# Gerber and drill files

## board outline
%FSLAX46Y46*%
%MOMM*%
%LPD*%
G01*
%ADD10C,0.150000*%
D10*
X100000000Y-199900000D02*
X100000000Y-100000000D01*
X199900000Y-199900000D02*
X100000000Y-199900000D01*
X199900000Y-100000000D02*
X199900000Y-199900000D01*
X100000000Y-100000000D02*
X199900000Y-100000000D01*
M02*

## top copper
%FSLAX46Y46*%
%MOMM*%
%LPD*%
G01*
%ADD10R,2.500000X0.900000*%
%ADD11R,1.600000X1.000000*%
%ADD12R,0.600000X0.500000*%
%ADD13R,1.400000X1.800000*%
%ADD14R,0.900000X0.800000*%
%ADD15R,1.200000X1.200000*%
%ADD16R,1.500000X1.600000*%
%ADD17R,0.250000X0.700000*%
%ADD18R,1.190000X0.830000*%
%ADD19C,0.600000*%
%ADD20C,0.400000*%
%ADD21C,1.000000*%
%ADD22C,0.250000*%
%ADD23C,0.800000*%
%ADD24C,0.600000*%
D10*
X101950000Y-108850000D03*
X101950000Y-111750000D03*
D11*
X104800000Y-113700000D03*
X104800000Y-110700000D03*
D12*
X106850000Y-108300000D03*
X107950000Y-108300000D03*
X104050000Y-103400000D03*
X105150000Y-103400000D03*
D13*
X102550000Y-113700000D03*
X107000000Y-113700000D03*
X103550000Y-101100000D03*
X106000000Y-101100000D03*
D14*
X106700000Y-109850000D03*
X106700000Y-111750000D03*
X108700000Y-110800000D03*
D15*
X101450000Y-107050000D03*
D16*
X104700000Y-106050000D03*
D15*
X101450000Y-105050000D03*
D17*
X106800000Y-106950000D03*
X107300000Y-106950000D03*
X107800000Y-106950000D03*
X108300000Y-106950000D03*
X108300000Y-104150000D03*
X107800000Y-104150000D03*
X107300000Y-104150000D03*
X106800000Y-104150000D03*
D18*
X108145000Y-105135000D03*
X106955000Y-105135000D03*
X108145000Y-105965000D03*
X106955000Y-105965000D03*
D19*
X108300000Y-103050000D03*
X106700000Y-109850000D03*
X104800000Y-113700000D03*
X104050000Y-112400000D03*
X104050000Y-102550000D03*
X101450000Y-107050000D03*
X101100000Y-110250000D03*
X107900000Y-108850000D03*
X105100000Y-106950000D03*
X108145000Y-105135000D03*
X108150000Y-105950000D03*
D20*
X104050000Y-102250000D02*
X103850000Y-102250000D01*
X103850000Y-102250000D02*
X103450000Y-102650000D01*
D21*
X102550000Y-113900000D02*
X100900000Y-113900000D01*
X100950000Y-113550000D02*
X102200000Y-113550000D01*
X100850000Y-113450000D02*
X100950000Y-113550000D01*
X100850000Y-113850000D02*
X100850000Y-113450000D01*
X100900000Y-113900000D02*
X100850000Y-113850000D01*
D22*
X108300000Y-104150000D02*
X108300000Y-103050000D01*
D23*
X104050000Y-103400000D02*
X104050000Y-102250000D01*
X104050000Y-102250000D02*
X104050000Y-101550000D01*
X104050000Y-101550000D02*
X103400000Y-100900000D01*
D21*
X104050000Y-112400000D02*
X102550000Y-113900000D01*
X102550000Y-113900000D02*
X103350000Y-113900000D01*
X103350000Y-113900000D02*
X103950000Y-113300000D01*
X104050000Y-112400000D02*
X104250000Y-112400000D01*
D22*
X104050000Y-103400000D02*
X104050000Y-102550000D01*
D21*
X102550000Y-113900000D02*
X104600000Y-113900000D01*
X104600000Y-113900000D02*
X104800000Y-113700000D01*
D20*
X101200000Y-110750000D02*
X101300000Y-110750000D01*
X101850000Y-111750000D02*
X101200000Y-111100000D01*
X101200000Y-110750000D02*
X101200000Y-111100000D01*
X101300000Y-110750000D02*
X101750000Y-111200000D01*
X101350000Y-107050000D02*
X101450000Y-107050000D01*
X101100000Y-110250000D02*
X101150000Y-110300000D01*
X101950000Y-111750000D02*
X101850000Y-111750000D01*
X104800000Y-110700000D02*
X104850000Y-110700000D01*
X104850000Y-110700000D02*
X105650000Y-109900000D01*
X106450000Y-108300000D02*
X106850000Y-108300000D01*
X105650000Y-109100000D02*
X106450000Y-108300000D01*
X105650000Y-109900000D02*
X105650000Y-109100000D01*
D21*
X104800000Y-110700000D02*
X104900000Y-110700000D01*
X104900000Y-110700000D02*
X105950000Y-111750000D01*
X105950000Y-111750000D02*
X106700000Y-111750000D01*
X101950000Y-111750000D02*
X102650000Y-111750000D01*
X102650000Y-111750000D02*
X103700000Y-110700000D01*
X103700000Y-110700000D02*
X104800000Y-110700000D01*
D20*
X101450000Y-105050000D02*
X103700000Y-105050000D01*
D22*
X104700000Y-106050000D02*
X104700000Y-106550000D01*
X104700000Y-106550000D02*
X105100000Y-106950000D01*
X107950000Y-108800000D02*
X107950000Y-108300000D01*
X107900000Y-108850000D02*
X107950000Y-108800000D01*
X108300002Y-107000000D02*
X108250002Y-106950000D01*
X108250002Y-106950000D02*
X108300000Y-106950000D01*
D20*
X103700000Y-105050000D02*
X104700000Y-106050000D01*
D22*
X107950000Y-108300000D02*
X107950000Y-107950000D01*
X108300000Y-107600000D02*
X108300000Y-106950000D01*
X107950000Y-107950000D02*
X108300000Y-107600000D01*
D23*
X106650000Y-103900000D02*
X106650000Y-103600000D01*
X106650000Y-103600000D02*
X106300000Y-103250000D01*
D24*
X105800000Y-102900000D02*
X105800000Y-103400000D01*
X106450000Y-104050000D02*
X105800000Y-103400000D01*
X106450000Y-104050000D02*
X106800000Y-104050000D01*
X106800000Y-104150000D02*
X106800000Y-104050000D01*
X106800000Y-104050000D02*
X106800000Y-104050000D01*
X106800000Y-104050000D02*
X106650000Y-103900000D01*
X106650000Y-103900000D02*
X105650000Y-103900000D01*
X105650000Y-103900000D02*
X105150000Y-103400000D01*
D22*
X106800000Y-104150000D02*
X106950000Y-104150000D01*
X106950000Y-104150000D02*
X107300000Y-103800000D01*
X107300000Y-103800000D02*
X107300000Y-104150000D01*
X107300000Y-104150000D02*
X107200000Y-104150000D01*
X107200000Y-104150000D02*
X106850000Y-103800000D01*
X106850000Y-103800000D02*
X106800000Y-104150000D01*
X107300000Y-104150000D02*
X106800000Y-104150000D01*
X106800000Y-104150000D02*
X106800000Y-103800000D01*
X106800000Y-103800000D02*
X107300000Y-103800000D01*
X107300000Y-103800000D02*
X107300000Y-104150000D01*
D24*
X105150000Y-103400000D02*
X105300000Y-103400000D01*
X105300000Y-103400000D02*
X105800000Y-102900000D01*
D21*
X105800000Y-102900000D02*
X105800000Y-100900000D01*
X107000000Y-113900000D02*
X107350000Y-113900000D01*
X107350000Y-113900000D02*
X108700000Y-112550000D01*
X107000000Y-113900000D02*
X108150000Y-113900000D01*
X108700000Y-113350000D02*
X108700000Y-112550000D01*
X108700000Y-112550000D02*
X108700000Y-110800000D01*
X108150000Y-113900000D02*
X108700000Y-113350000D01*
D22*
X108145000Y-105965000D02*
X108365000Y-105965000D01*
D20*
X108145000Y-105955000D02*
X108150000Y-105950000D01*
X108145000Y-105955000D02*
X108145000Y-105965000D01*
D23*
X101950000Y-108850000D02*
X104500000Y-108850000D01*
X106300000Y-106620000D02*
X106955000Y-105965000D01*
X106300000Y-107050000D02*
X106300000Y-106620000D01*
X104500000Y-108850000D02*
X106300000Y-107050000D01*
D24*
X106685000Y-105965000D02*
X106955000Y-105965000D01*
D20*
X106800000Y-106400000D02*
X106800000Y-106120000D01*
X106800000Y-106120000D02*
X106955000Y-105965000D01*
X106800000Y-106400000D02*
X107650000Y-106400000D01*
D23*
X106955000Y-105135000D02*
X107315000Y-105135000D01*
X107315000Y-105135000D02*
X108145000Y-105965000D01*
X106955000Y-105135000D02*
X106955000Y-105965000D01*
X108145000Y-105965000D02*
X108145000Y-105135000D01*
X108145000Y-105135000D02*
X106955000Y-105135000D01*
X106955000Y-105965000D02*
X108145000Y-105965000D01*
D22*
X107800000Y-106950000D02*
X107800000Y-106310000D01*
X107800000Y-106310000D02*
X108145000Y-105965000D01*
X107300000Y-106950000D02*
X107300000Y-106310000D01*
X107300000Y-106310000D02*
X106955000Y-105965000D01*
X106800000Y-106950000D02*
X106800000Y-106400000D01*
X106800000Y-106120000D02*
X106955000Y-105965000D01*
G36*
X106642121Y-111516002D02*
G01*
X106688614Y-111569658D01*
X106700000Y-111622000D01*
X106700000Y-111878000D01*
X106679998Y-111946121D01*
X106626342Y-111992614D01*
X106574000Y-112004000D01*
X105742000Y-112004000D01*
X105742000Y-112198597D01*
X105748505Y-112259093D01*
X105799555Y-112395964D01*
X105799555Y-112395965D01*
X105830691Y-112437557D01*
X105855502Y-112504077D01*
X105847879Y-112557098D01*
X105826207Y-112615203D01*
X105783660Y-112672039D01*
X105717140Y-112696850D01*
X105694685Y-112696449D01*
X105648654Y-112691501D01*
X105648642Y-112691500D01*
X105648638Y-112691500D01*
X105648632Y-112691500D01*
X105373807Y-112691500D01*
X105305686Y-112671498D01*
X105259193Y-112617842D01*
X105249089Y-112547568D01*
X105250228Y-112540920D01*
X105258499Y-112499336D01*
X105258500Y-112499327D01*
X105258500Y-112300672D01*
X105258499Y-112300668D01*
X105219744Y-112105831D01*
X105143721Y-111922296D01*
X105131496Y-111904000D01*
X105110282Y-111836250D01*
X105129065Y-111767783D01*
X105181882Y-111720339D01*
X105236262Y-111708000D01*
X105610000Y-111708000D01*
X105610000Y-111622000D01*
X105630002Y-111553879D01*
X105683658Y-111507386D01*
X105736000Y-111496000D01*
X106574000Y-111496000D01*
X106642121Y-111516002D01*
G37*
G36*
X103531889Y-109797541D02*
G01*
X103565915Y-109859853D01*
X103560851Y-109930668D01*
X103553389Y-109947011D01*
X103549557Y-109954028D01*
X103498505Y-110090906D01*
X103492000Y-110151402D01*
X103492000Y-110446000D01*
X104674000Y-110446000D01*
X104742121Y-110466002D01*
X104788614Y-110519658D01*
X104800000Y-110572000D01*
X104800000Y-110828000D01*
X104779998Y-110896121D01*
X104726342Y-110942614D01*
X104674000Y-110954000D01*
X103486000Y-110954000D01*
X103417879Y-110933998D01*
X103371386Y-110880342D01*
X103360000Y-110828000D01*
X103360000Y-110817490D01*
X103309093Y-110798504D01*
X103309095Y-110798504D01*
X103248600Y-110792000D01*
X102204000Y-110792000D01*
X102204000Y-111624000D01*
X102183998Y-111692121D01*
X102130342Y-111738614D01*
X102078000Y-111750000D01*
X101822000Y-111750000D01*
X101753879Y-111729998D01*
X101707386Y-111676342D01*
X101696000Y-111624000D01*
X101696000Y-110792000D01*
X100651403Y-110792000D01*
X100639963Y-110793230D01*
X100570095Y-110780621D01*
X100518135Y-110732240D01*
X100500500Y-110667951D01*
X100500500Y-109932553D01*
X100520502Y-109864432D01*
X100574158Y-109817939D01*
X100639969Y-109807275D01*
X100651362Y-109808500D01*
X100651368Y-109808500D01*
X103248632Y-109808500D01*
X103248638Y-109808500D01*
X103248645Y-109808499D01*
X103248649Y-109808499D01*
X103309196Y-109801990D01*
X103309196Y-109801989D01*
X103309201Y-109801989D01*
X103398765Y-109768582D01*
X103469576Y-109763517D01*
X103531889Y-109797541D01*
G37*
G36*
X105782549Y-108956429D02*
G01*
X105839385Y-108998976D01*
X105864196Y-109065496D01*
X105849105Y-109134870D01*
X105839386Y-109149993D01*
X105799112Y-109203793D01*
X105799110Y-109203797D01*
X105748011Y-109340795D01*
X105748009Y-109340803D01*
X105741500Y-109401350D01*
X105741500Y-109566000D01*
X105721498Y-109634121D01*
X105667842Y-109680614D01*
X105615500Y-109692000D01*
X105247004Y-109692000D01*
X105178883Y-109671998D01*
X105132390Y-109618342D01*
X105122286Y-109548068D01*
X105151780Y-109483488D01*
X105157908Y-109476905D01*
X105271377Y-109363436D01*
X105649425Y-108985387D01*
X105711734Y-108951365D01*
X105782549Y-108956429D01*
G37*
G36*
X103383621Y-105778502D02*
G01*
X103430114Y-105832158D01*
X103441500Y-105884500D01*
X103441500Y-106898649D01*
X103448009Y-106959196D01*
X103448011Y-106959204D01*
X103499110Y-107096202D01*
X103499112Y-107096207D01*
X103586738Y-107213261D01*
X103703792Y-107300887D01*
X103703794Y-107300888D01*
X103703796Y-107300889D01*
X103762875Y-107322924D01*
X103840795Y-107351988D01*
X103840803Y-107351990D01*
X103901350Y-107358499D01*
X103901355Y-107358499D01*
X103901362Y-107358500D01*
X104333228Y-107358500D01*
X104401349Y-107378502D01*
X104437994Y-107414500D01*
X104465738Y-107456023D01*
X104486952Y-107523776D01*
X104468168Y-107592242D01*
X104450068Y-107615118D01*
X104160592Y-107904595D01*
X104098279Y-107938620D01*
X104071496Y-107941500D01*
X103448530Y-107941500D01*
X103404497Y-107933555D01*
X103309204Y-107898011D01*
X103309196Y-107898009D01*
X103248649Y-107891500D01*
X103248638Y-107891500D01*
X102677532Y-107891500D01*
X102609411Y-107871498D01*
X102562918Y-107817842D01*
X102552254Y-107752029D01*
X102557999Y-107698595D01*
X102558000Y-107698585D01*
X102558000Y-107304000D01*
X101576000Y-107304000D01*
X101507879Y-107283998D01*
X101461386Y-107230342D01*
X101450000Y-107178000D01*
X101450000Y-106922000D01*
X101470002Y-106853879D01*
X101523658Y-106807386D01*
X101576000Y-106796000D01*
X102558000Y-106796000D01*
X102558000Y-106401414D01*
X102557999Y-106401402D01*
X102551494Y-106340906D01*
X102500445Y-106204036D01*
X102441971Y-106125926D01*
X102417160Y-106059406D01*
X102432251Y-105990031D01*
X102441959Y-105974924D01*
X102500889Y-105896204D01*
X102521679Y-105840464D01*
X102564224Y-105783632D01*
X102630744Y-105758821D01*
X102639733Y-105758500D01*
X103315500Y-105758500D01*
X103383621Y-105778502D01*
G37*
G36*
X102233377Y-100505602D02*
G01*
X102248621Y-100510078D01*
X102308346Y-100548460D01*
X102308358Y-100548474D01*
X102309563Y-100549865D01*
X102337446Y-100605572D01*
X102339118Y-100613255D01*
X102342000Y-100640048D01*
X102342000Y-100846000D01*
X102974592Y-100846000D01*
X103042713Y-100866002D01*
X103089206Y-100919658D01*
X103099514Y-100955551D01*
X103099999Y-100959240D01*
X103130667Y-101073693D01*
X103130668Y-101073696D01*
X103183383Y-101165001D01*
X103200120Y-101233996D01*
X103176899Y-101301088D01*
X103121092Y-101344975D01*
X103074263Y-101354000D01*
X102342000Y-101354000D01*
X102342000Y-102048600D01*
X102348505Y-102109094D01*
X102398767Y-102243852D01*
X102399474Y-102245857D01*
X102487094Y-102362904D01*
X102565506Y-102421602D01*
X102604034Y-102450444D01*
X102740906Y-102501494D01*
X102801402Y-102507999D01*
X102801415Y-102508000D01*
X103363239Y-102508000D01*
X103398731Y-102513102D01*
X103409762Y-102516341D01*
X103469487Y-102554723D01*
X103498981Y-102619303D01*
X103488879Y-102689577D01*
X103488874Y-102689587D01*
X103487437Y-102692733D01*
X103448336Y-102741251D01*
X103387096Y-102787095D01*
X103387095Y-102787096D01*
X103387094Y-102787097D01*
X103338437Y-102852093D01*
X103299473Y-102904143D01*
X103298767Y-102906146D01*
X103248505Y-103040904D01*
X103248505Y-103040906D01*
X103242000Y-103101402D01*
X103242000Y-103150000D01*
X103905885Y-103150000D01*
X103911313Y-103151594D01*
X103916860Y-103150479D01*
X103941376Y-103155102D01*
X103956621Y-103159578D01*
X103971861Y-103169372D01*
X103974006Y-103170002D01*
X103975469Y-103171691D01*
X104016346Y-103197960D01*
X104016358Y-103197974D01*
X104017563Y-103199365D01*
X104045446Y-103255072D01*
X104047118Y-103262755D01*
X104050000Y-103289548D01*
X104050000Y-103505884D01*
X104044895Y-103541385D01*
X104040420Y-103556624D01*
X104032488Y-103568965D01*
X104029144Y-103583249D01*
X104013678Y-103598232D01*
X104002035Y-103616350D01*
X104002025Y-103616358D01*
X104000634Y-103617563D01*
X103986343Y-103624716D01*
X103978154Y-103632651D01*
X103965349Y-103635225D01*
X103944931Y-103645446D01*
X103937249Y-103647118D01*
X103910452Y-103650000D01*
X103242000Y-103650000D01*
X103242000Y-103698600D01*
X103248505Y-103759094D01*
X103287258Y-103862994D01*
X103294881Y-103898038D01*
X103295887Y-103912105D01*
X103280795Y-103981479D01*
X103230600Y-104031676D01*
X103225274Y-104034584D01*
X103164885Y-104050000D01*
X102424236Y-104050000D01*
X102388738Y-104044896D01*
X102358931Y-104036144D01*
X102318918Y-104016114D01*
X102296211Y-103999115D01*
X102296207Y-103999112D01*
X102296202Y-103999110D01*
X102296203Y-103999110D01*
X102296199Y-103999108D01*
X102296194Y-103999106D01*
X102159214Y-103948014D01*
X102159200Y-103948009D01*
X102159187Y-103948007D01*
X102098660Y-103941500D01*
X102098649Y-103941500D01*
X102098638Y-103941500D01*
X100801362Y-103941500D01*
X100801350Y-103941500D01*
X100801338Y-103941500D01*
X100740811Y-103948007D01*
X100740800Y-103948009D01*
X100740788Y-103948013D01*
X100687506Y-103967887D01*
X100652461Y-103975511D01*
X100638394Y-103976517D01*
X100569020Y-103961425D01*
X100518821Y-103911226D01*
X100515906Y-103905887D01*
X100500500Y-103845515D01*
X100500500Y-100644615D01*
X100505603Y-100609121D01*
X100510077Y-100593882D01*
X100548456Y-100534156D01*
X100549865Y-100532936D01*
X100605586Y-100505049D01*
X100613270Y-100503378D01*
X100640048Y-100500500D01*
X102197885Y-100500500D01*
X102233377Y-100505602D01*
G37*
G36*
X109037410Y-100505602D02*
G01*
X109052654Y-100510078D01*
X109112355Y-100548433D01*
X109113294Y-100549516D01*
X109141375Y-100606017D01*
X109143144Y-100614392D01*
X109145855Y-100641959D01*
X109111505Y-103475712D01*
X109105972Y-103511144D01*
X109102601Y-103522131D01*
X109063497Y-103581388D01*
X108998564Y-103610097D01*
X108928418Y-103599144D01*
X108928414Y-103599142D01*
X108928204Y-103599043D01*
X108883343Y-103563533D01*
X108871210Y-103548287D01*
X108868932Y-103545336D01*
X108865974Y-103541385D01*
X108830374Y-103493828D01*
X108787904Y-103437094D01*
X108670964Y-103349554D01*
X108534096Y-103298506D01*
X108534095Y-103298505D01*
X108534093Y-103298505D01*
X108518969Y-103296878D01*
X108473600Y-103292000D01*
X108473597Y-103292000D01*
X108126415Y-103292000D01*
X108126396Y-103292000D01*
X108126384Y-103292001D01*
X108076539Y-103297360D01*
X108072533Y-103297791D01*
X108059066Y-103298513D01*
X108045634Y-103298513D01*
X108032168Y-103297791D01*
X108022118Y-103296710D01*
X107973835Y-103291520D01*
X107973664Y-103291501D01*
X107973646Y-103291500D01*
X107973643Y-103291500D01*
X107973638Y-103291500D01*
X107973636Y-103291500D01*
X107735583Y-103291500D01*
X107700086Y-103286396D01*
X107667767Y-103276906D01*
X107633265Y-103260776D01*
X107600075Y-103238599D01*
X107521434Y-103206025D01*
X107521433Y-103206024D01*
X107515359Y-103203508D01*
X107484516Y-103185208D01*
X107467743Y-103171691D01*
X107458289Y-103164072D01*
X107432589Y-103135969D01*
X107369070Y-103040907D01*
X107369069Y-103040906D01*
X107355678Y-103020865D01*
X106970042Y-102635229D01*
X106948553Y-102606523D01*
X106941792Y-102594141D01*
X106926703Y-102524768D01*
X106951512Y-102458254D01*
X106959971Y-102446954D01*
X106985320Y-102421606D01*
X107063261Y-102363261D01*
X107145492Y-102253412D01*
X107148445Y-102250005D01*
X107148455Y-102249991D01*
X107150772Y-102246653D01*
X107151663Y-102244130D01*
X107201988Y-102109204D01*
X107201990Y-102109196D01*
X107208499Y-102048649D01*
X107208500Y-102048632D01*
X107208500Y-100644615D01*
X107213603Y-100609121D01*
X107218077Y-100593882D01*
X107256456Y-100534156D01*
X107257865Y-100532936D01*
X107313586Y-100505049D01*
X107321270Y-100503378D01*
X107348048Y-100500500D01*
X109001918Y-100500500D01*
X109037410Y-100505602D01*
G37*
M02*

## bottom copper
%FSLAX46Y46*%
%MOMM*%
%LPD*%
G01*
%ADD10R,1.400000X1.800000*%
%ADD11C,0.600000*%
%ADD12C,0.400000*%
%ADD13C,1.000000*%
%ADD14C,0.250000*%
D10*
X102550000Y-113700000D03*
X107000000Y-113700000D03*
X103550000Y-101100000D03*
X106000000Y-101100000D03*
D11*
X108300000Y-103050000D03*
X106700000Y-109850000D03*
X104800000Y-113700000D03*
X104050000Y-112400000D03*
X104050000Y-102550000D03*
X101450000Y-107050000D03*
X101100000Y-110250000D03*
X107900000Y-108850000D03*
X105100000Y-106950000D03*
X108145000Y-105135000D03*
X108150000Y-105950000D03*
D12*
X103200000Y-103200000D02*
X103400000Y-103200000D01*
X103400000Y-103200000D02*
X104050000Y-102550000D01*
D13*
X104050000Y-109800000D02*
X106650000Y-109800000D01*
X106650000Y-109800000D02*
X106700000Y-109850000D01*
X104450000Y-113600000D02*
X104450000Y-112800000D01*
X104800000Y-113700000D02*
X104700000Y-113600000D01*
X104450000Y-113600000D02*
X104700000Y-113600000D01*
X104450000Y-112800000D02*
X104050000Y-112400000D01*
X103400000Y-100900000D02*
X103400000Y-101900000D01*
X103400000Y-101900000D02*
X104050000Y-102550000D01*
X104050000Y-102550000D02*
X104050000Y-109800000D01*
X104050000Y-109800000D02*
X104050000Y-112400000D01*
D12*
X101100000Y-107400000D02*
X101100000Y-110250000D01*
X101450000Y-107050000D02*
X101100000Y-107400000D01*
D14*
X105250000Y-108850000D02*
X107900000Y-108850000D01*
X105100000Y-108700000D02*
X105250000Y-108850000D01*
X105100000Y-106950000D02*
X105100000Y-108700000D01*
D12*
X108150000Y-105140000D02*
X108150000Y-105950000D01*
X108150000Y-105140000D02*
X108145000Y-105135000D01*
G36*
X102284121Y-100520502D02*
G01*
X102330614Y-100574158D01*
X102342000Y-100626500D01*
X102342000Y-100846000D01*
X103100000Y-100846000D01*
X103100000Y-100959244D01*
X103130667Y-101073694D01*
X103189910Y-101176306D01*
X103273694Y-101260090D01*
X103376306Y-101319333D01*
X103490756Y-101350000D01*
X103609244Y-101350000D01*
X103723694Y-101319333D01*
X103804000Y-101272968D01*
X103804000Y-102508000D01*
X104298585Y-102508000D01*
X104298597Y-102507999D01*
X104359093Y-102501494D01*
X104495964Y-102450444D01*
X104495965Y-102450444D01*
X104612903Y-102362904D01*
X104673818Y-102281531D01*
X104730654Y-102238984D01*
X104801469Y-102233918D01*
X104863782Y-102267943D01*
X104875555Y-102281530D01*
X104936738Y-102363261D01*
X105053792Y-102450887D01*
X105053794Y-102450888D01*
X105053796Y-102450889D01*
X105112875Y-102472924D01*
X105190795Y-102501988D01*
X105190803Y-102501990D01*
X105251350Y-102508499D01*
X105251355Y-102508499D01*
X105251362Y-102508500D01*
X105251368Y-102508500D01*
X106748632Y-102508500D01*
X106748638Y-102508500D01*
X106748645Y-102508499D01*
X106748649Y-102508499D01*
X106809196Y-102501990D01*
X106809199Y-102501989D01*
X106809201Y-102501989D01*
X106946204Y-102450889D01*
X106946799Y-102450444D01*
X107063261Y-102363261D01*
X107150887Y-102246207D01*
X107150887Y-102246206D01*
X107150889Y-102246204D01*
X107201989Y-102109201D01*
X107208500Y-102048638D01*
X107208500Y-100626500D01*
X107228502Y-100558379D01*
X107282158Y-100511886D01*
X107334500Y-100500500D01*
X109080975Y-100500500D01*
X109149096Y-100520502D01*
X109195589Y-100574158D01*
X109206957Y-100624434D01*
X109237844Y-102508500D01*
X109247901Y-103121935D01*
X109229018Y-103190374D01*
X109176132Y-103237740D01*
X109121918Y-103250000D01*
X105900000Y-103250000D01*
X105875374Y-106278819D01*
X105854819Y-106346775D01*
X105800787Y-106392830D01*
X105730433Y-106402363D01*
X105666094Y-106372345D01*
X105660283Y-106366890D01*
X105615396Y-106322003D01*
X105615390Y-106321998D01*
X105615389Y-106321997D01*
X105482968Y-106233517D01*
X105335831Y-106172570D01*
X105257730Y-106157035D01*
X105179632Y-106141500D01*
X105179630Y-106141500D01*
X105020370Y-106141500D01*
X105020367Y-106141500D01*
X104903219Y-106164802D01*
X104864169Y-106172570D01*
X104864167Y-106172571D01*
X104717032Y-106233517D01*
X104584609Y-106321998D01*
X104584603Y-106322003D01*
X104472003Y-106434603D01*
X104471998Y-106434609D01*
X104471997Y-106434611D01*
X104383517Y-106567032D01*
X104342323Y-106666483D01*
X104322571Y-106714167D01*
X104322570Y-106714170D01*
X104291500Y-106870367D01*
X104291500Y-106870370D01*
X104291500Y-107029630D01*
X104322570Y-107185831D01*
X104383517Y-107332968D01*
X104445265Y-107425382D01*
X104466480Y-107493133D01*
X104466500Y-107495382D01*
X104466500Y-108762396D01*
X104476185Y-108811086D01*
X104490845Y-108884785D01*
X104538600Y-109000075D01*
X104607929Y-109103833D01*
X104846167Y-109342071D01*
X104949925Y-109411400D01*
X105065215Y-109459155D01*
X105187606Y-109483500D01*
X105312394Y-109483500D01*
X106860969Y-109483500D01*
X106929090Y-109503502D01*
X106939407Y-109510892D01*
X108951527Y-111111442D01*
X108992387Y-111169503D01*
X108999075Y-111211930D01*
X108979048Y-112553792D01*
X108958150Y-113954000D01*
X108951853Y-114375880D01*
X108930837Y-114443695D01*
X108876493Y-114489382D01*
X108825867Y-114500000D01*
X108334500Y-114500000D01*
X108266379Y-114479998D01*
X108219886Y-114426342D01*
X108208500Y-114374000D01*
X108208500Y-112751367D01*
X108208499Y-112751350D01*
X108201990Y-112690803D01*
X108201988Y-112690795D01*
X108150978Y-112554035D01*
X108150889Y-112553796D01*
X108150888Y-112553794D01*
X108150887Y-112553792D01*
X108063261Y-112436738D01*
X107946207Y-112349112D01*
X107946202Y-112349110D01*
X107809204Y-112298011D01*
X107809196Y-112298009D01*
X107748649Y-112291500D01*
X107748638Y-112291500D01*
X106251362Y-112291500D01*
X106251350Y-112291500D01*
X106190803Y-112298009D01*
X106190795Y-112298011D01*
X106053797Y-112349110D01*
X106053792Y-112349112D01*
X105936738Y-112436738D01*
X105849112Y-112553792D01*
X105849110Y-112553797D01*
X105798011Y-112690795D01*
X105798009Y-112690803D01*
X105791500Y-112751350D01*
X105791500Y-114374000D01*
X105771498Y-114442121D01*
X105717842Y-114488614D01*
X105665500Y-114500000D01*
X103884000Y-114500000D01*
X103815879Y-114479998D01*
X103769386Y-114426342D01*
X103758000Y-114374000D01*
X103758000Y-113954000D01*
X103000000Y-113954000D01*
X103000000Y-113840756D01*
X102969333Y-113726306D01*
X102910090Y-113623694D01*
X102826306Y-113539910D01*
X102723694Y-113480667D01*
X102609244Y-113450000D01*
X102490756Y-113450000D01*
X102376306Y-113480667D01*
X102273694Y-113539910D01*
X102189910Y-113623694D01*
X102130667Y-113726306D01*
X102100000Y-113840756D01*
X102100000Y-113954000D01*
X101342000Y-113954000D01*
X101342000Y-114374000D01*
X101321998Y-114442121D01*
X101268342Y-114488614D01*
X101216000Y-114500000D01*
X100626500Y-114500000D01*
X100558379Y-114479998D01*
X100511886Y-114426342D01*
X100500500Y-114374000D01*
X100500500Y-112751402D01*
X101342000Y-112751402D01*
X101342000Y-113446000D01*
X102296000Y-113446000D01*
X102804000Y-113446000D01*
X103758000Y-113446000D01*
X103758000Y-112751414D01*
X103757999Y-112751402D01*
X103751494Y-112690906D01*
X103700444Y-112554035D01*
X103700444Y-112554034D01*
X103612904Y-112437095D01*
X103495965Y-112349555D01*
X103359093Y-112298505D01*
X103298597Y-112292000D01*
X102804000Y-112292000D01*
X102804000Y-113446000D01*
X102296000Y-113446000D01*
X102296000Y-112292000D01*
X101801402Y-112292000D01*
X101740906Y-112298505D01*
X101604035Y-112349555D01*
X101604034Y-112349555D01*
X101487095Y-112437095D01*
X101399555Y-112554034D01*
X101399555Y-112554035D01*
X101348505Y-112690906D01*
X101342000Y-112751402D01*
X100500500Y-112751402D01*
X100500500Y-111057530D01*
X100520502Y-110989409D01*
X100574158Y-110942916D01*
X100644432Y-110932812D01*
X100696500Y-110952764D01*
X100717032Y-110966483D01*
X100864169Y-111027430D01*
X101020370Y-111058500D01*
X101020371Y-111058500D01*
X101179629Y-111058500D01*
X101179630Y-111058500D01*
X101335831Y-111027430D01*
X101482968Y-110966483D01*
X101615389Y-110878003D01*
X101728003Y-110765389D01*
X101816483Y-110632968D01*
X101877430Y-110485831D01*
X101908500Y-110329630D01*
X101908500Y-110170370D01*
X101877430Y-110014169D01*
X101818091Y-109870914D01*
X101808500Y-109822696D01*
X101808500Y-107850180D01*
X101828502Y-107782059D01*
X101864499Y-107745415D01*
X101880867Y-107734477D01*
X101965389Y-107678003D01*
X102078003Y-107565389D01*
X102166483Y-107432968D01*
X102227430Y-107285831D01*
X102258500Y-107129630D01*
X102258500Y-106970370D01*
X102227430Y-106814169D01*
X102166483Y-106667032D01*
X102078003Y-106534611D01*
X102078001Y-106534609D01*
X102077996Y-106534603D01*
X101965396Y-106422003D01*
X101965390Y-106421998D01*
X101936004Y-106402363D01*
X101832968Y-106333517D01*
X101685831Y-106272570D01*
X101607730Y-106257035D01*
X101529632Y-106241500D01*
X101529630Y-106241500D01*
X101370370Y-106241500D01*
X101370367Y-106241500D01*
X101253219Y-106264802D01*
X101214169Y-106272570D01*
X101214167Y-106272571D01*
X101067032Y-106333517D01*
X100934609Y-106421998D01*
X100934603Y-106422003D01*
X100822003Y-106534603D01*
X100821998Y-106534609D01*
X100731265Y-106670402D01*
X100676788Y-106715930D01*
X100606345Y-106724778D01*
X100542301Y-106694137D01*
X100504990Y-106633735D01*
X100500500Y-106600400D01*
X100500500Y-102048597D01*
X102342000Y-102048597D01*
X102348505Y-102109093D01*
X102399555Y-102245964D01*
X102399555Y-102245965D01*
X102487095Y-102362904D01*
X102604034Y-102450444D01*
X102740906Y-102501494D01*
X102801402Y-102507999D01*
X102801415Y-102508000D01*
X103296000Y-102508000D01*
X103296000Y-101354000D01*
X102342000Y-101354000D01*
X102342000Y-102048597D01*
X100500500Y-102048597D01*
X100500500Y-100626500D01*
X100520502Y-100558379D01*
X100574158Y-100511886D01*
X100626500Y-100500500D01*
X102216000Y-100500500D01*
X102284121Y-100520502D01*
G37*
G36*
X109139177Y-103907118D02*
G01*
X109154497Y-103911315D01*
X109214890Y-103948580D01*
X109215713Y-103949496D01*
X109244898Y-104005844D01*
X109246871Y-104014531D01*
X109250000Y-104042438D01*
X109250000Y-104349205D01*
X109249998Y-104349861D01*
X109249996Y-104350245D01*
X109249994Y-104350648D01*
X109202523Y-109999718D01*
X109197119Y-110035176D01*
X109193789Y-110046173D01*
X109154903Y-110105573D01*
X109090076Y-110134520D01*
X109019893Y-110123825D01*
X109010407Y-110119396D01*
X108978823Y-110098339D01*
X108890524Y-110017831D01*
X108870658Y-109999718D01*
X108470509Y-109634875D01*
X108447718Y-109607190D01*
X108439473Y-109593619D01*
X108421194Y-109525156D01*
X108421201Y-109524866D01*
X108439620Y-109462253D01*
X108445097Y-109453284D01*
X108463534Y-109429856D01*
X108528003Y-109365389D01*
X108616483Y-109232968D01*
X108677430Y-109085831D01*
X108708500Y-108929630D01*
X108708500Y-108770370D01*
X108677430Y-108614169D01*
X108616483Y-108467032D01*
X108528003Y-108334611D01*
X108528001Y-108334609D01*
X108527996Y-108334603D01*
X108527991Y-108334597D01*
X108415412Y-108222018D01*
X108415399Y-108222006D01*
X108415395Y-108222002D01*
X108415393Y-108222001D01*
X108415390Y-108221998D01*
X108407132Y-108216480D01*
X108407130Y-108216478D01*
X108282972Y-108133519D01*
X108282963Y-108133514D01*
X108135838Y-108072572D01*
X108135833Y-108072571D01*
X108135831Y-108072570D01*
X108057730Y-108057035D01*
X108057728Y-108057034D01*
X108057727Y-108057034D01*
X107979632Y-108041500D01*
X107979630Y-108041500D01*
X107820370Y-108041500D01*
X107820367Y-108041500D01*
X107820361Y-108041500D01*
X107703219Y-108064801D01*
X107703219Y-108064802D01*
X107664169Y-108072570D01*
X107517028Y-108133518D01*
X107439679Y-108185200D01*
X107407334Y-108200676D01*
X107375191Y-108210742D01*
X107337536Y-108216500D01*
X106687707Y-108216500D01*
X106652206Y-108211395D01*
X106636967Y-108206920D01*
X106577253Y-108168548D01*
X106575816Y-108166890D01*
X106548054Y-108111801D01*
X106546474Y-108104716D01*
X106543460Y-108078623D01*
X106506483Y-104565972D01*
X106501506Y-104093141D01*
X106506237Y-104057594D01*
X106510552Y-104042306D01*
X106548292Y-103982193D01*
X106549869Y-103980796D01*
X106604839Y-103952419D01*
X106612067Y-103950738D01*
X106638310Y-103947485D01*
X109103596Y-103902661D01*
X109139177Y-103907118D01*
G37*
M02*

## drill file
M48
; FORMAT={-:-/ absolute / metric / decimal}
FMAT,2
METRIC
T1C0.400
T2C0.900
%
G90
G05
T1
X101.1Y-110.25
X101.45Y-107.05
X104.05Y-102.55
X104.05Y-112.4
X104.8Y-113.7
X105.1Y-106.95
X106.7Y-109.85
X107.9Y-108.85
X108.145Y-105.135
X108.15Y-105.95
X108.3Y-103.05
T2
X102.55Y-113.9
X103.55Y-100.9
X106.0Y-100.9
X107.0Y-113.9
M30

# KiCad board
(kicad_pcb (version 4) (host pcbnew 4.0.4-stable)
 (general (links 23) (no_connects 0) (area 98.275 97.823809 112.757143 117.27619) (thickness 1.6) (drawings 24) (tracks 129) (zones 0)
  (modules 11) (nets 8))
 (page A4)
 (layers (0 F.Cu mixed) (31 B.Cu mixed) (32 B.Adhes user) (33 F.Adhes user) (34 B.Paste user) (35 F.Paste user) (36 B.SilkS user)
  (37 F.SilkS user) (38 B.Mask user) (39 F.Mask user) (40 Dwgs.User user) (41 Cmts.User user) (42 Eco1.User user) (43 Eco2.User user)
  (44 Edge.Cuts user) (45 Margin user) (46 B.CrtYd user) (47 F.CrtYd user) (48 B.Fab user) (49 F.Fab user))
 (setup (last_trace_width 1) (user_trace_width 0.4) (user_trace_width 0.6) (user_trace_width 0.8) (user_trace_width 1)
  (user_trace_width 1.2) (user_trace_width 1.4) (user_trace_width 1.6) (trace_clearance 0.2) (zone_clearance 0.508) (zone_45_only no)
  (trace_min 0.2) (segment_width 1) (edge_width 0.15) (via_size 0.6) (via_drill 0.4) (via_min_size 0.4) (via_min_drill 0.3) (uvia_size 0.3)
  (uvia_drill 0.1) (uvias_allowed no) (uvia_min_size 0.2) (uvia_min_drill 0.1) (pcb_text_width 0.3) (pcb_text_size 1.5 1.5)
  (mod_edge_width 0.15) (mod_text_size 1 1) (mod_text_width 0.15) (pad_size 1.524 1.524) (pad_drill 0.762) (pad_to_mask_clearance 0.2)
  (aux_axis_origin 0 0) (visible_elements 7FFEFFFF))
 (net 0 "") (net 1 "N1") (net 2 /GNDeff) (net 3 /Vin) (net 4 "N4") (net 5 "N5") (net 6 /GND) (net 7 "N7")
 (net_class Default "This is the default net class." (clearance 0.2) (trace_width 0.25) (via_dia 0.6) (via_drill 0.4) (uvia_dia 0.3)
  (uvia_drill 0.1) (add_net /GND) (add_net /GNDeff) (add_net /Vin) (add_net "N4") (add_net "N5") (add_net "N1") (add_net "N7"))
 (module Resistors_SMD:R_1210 (layer F.Cu) (at 101.95 110.3 270)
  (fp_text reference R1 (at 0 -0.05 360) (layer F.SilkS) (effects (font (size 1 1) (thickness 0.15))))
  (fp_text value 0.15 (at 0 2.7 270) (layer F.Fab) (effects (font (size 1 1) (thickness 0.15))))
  (pad 1 smd rect (at -1.45 0 270) (size 0.9 2.5) (layers F.Cu F.Paste F.Mask) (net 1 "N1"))
  (pad 2 smd rect (at 1.45 0 270) (size 0.9 2.5) (layers F.Cu F.Paste F.Mask) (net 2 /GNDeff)))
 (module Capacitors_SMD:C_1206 (layer F.Cu) (at 104.8 112.2 90)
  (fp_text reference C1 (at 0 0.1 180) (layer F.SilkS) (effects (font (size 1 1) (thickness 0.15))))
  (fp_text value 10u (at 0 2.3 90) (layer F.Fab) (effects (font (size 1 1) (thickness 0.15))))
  (pad 1 smd rect (at -1.5 0 90) (size 1 1.6) (layers F.Cu F.Paste F.Mask) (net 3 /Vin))
  (pad 2 smd rect (at 1.5 0 90) (size 1 1.6) (layers F.Cu F.Paste F.Mask) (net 2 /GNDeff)))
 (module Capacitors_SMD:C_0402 (layer F.Cu) (at 107.4 108.3)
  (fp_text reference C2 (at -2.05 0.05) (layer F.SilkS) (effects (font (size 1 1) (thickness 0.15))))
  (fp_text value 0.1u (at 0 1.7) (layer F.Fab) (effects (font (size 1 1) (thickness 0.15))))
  (pad 1 smd rect (at -0.55 0) (size 0.6 0.5) (layers F.Cu F.Paste F.Mask) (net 2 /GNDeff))
  (pad 2 smd rect (at 0.55 0) (size 0.6 0.5) (layers F.Cu F.Paste F.Mask) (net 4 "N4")))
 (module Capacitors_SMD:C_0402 (layer F.Cu) (at 104.6 103.4)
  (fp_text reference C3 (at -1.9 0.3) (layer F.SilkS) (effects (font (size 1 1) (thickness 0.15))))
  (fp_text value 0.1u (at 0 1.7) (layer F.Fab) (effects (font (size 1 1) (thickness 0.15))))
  (pad 1 smd rect (at -0.55 0) (size 0.6 0.5) (layers F.Cu F.Paste F.Mask) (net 3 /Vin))
  (pad 2 smd rect (at 0.55 0) (size 0.6 0.5) (layers F.Cu F.Paste F.Mask) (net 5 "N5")))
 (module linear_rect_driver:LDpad (layer F.Cu) (at 103 113.85 270)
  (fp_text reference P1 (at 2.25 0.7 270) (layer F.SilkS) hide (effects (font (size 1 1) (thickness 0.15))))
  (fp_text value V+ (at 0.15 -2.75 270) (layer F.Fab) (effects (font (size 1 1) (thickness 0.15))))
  (pad 1 thru_hole rect (at 0.05 0.45 270) (size 1.8 1.4) (drill 0.9 (offset -0.2 0)) (layers *.Cu *.Mask) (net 3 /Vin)))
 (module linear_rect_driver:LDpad (layer F.Cu) (at 107.45 113.85 270)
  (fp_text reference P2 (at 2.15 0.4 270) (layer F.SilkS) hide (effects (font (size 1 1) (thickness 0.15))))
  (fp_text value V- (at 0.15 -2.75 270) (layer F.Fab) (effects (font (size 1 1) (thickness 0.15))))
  (pad 1 thru_hole rect (at 0.05 0.45 270) (size 1.8 1.4) (drill 0.9 (offset -0.2 0)) (layers *.Cu *.Mask) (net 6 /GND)))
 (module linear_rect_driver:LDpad (layer F.Cu) (at 103.1 100.95 90)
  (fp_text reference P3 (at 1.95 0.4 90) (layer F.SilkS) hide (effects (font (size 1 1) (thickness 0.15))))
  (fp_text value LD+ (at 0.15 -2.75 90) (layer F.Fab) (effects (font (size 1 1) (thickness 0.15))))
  (pad 1 thru_hole rect (at 0.05 0.45 90) (size 1.8 1.4) (drill 0.9 (offset -0.2 0)) (layers *.Cu *.Mask) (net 3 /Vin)))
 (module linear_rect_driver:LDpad (layer F.Cu) (at 105.55 100.95 90)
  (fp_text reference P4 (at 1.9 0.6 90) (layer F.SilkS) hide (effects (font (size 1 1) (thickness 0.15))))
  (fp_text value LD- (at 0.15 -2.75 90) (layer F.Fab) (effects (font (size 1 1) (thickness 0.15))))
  (pad 1 thru_hole rect (at 0.05 0.45 90) (size 1.8 1.4) (drill 0.9 (offset -0.2 0)) (layers *.Cu *.Mask) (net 5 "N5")))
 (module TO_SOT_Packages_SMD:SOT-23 (layer F.Cu) (at 107.7 110.8)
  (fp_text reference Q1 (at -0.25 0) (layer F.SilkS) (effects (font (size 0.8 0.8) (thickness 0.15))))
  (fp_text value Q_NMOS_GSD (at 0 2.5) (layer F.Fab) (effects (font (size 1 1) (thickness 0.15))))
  (pad 1 smd rect (at -1 -0.95) (size 0.9 0.8) (layers F.Cu F.Paste F.Mask) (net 3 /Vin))
  (pad 2 smd rect (at -1 0.95) (size 0.9 0.8) (layers F.Cu F.Paste F.Mask) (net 2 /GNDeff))
  (pad 3 smd rect (at 1 0) (size 0.9 0.8) (layers F.Cu F.Paste F.Mask) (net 6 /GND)))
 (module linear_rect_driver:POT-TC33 (layer F.Cu) (at 103.95 106.05 270)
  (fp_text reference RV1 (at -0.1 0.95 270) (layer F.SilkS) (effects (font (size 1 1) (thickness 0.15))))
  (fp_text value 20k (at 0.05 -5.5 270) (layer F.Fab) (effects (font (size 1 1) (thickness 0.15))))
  (pad 3 smd rect (at 1 2.5 270) (size 1.2 1.2) (layers F.Cu F.Paste F.Mask) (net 2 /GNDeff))
  (pad 2 smd rect (at 0 -0.75 270) (size 1.6 1.5) (layers F.Cu F.Paste F.Mask) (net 4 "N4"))
  (pad 1 smd rect (at -1 2.5 270) (size 1.2 1.2) (layers F.Cu F.Paste F.Mask) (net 4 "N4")))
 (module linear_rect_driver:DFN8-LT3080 (layer F.Cu) (at 107.55 105.55 90)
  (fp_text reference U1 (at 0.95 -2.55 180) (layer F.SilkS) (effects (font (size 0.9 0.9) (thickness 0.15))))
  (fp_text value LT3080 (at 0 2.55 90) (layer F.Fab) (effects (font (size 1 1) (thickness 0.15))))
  (pad 1 smd rect (at -1.4 -0.75 90) (size 0.7 0.25) (layers F.Cu F.Paste F.Mask) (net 1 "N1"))
  (pad 1 smd rect (at -1.4 -0.25 90) (size 0.7 0.25) (layers F.Cu F.Paste F.Mask) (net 1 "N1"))
  (pad 1 smd rect (at -1.4 0.25 90) (size 0.7 0.25) (layers F.Cu F.Paste F.Mask) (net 1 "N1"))
  (pad 2 smd rect (at -1.4 0.75 90) (size 0.7 0.25) (layers F.Cu F.Paste F.Mask) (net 4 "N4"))
  (pad 3 smd rect (at 1.4 0.75 90) (size 0.7 0.25) (layers F.Cu F.Paste F.Mask) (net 3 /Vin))
  (pad 5 smd rect (at 1.4 0.25 90) (size 0.7 0.25) (layers F.Cu F.Paste F.Mask) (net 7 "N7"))
  (pad 4 smd rect (at 1.4 -0.25 90) (size 0.7 0.25) (layers F.Cu F.Paste F.Mask) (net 5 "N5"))
  (pad 4 smd rect (at 1.4 -0.75 90) (size 0.7 0.25) (layers F.Cu F.Paste F.Mask) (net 5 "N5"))
  (pad 1 smd rect (at 0.415 0.595 90) (size 0.83 1.19) (layers F.Cu F.Paste F.Mask) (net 1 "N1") (solder_paste_margin_ratio -0.2))
  (pad 1 smd rect (at 0.415 -0.595 90) (size 0.83 1.19) (layers F.Cu F.Paste F.Mask) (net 1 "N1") (solder_paste_margin_ratio -0.2))
  (pad 1 smd rect (at -0.415 0.595 90) (size 0.83 1.19) (layers F.Cu F.Paste F.Mask) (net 1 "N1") (solder_paste_margin_ratio -0.2))
  (pad 1 smd rect (at -0.415 -0.595 90) (size 0.83 1.19) (layers F.Cu F.Paste F.Mask) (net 1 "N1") (solder_paste_margin_ratio -0.2)))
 (gr_line (start 100 199.9) (end 100 100) (angle 90) (layer Edge.Cuts) (width 0.15))
 (gr_line (start 199.9 199.9) (end 100 199.9) (angle 90) (layer Edge.Cuts) (width 0.15))
 (gr_line (start 199.9 100) (end 199.9 199.9) (angle 90) (layer Edge.Cuts) (width 0.15))
 (gr_line (start 100 100) (end 199.9 100) (angle 90) (layer Edge.Cuts) (width 0.15))
 (segment (start 104.05 102.25) (end 103.85 102.25) (width 0.4) (layer F.Cu) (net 3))
 (segment (start 103.85 102.25) (end 103.45 102.65) (width 0.4) (layer F.Cu) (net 3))
 (segment (start 103.2 103.2) (end 103.4 103.2) (width 0.4) (layer B.Cu) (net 3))
 (segment (start 103.4 103.2) (end 104.05 102.55) (width 0.4) (layer B.Cu) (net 3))
 (segment (start 102.55 113.9) (end 100.9 113.9) (width 1) (layer F.Cu) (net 3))
 (segment (start 100.95 113.55) (end 102.2 113.55) (width 1) (layer F.Cu) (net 3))
 (segment (start 100.85 113.45) (end 100.95 113.55) (width 1) (layer F.Cu) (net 3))
 (segment (start 100.85 113.85) (end 100.85 113.45) (width 1) (layer F.Cu) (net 3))
 (segment (start 100.9 113.9) (end 100.85 113.85) (width 1) (layer F.Cu) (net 3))
 (segment (start 108.3 104.15) (end 108.3 103.05) (width 0.25) (layer F.Cu) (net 3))
 (via (at 108.3 103.05) (size 0.6) (drill 0.4) (layers F.Cu B.Cu) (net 3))
 (segment (start 104.05 103.4) (end 104.05 102.25) (width 0.8) (layer F.Cu) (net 3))
 (segment (start 104.05 102.25) (end 104.05 101.55) (width 0.8) (layer F.Cu) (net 3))
 (segment (start 104.05 101.55) (end 103.4 100.9) (width 0.8) (layer F.Cu) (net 3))
 (via (at 106.7 109.85) (size 0.6) (drill 0.4) (layers F.Cu B.Cu) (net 3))
 (segment (start 104.05 109.8) (end 106.65 109.8) (width 1) (layer B.Cu) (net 3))
 (segment (start 106.65 109.8) (end 106.7 109.85) (width 1) (layer B.Cu) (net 3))
 (segment (start 104.45 113.6) (end 104.45 112.8) (width 1) (layer B.Cu) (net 3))
 (segment (start 104.8 113.7) (end 104.7 113.6) (width 1) (layer B.Cu) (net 3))
 (segment (start 104.45 113.6) (end 104.7 113.6) (width 1) (layer B.Cu) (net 3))
 (via (at 104.8 113.7) (size 0.6) (drill 0.4) (layers F.Cu B.Cu) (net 3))
 (segment (start 104.45 112.8) (end 104.05 112.4) (width 1) (layer B.Cu) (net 3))
 (segment (start 104.05 112.4) (end 102.55 113.9) (width 1) (layer F.Cu) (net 3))
 (segment (start 102.55 113.9) (end 103.35 113.9) (width 1) (layer F.Cu) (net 3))
 (segment (start 103.35 113.9) (end 103.95 113.3) (width 1) (layer F.Cu) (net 3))
 (via (at 104.05 112.4) (size 0.6) (drill 0.4) (layers F.Cu B.Cu) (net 3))
 (segment (start 104.05 112.4) (end 104.25 112.4) (width 1) (layer F.Cu) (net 3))
 (segment (start 103.4 100.9) (end 103.4 101.9) (width 1) (layer B.Cu) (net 3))
 (segment (start 103.4 101.9) (end 104.05 102.55) (width 1) (layer B.Cu) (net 3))
 (segment (start 104.05 102.55) (end 104.05 109.8) (width 1) (layer B.Cu) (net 3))
 (segment (start 104.05 109.8) (end 104.05 112.4) (width 1) (layer B.Cu) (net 3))
 (via (at 104.05 102.55) (size 0.6) (drill 0.4) (layers F.Cu B.Cu) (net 3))
 (segment (start 104.05 103.4) (end 104.05 102.55) (width 0.25) (layer F.Cu) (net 3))
 (segment (start 102.55 113.9) (end 104.6 113.9) (width 1) (layer F.Cu) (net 3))
 (segment (start 104.6 113.9) (end 104.8 113.7) (width 1) (layer F.Cu) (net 3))
 (segment (start 101.2 110.75) (end 101.3 110.75) (width 0.4) (layer F.Cu) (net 2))
 (segment (start 101.85 111.75) (end 101.2 111.1) (width 0.4) (layer F.Cu) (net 2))
 (segment (start 101.2 110.75) (end 101.2 111.1) (width 0.4) (layer F.Cu) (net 2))
 (segment (start 101.3 110.75) (end 101.75 111.2) (width 0.4) (layer F.Cu) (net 2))
 (via (at 101.45 107.05) (size 0.6) (drill 0.4) (layers F.Cu B.Cu) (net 2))
 (segment (start 101.35 107.05) (end 101.45 107.05) (width 0.4) (layer F.Cu) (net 2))
 (segment (start 101.1 110.25) (end 101.15 110.3) (width 0.4) (layer F.Cu) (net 2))
 (via (at 101.1 110.25) (size 0.6) (drill 0.4) (layers F.Cu B.Cu) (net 2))
 (segment (start 101.1 107.4) (end 101.1 110.25) (width 0.4) (layer B.Cu) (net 2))
 (segment (start 101.45 107.05) (end 101.1 107.4) (width 0.4) (layer B.Cu) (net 2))
 (segment (start 101.95 111.75) (end 101.85 111.75) (width 0.4) (layer F.Cu) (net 2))
 (segment (start 104.8 110.7) (end 104.85 110.7) (width 0.4) (layer F.Cu) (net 2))
 (segment (start 104.85 110.7) (end 105.65 109.9) (width 0.4) (layer F.Cu) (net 2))
 (segment (start 106.45 108.3) (end 106.85 108.3) (width 0.4) (layer F.Cu) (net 2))
 (segment (start 105.65 109.1) (end 106.45 108.3) (width 0.4) (layer F.Cu) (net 2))
 (segment (start 105.65 109.9) (end 105.65 109.1) (width 0.4) (layer F.Cu) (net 2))
 (segment (start 104.8 110.7) (end 104.9 110.7) (width 1) (layer F.Cu) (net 2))
 (segment (start 104.9 110.7) (end 105.95 111.75) (width 1) (layer F.Cu) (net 2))
 (segment (start 105.95 111.75) (end 106.7 111.75) (width 1) (layer F.Cu) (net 2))
 (segment (start 101.95 111.75) (end 102.65 111.75) (width 1) (layer F.Cu) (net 2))
 (segment (start 102.65 111.75) (end 103.7 110.7) (width 1) (layer F.Cu) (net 2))
 (segment (start 103.7 110.7) (end 104.8 110.7) (width 1) (layer F.Cu) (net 2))
 (segment (start 101.45 105.05) (end 103.7 105.05) (width 0.4) (layer F.Cu) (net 4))
 (segment (start 104.7 106.05) (end 104.7 106.55) (width 0.25) (layer F.Cu) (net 4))
 (segment (start 104.7 106.55) (end 105.1 106.95) (width 0.25) (layer F.Cu) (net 4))
 (segment (start 107.95 108.8) (end 107.95 108.3) (width 0.25) (layer F.Cu) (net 4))
 (segment (start 107.9 108.85) (end 107.95 108.8) (width 0.25) (layer F.Cu) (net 4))
 (via (at 107.9 108.85) (size 0.6) (drill 0.4) (layers F.Cu B.Cu) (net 4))
 (segment (start 105.25 108.85) (end 107.9 108.85) (width 0.25) (layer B.Cu) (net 4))
 (segment (start 105.1 108.7) (end 105.25 108.85) (width 0.25) (layer B.Cu) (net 4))
 (segment (start 105.1 106.95) (end 105.1 108.7) (width 0.25) (layer B.Cu) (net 4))
 (via (at 105.1 106.95) (size 0.6) (drill 0.4) (layers F.Cu B.Cu) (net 4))
 (segment (start 108.300002 107) (end 108.250002 106.95) (width 0.25) (layer F.Cu) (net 4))
 (segment (start 108.250002 106.95) (end 108.3 106.95) (width 0.25) (layer F.Cu) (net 4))
 (segment (start 103.7 105.05) (end 104.7 106.05) (width 0.4) (layer F.Cu) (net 4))
 (segment (start 107.95 108.3) (end 107.95 107.95) (width 0.25) (layer F.Cu) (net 4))
 (segment (start 108.3 107.6) (end 108.3 106.95) (width 0.25) (layer F.Cu) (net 4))
 (segment (start 107.95 107.95) (end 108.3 107.6) (width 0.25) (layer F.Cu) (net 4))
 (segment (start 106.65 103.9) (end 106.65 103.6) (width 0.8) (layer F.Cu) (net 5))
 (segment (start 106.65 103.6) (end 106.3 103.25) (width 0.8) (layer F.Cu) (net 5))
 (segment (start 105.8 102.9) (end 105.8 103.4) (width 0.6) (layer F.Cu) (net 5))
 (segment (start 106.45 104.05) (end 105.8 103.4) (width 0.6) (layer F.Cu) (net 5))
 (segment (start 106.45 104.05) (end 106.8 104.05) (width 0.6) (layer F.Cu) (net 5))
 (segment (start 106.8 104.15) (end 106.8 104.05) (width 0.6) (layer F.Cu) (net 5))
 (segment (start 106.8 104.05) (end 106.8 104.05) (width 0.6) (layer F.Cu) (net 5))
 (segment (start 106.8 104.05) (end 106.65 103.9) (width 0.6) (layer F.Cu) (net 5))
 (segment (start 106.65 103.9) (end 105.65 103.9) (width 0.6) (layer F.Cu) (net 5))
 (segment (start 105.65 103.9) (end 105.15 103.4) (width 0.6) (layer F.Cu) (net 5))
 (segment (start 106.8 104.15) (end 106.95 104.15) (width 0.25) (layer F.Cu) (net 5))
 (segment (start 106.95 104.15) (end 107.3 103.8) (width 0.25) (layer F.Cu) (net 5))
 (segment (start 107.3 103.8) (end 107.3 104.15) (width 0.25) (layer F.Cu) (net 5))
 (segment (start 107.3 104.15) (end 107.2 104.15) (width 0.25) (layer F.Cu) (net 5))
 (segment (start 107.2 104.15) (end 106.85 103.8) (width 0.25) (layer F.Cu) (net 5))
 (segment (start 106.85 103.8) (end 106.8 104.15) (width 0.25) (layer F.Cu) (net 5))
 (segment (start 107.3 104.15) (end 106.8 104.15) (width 0.25) (layer F.Cu) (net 5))
 (segment (start 106.8 104.15) (end 106.8 103.8) (width 0.25) (layer F.Cu) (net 5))
 (segment (start 106.8 103.8) (end 107.3 103.8) (width 0.25) (layer F.Cu) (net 5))
 (segment (start 107.3 103.8) (end 107.3 104.15) (width 0.25) (layer F.Cu) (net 5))
 (segment (start 105.15 103.4) (end 105.3 103.4) (width 0.6) (layer F.Cu) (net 5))
 (segment (start 105.3 103.4) (end 105.8 102.9) (width 0.6) (layer F.Cu) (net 5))
 (segment (start 105.8 102.9) (end 105.8 100.9) (width 1) (layer F.Cu) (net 5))
 (segment (start 107 113.9) (end 107.35 113.9) (width 1) (layer F.Cu) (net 6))
 (segment (start 107.35 113.9) (end 108.7 112.55) (width 1) (layer F.Cu) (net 6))
 (segment (start 107 113.9) (end 108.15 113.9) (width 1) (layer F.Cu) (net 6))
 (segment (start 108.7 113.35) (end 108.7 112.55) (width 1) (layer F.Cu) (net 6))
 (segment (start 108.7 112.55) (end 108.7 110.8) (width 1) (layer F.Cu) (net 6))
 (segment (start 108.15 113.9) (end 108.7 113.35) (width 1) (layer F.Cu) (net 6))
 (segment (start 108.145 105.965) (end 108.365 105.965) (width 0.25) (layer F.Cu) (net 1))
 (via (at 108.145 105.135) (size 0.6) (drill 0.4) (layers F.Cu B.Cu) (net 1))
 (segment (start 108.145 105.955) (end 108.15 105.95) (width 0.4) (layer F.Cu) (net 1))
 (via (at 108.15 105.95) (size 0.6) (drill 0.4) (layers F.Cu B.Cu) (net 1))
 (segment (start 108.15 105.14) (end 108.15 105.95) (width 0.4) (layer B.Cu) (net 1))
 (segment (start 108.15 105.14) (end 108.145 105.135) (width 0.4) (layer B.Cu) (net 1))
 (segment (start 108.145 105.955) (end 108.145 105.965) (width 0.4) (layer F.Cu) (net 1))
 (segment (start 101.95 108.85) (end 104.5 108.85) (width 0.8) (layer F.Cu) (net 1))
 (segment (start 106.3 106.62) (end 106.955 105.965) (width 0.8) (layer F.Cu) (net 1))
 (segment (start 106.3 107.05) (end 106.3 106.62) (width 0.8) (layer F.Cu) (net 1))
 (segment (start 104.5 108.85) (end 106.3 107.05) (width 0.8) (layer F.Cu) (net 1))
 (segment (start 106.685 105.965) (end 106.955 105.965) (width 0.6) (layer F.Cu) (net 1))
 (segment (start 106.8 106.4) (end 106.8 106.12) (width 0.4) (layer F.Cu) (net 1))
 (segment (start 106.8 106.12) (end 106.955 105.965) (width 0.4) (layer F.Cu) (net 1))
 (segment (start 106.8 106.4) (end 107.65 106.4) (width 0.4) (layer F.Cu) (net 1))
 (segment (start 106.955 105.135) (end 107.315 105.135) (width 0.8) (layer F.Cu) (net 1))
 (segment (start 107.315 105.135) (end 108.145 105.965) (width 0.8) (layer F.Cu) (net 1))
 (segment (start 106.955 105.135) (end 106.955 105.965) (width 0.8) (layer F.Cu) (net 1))
 (segment (start 108.145 105.965) (end 108.145 105.135) (width 0.8) (layer F.Cu) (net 1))
 (segment (start 108.145 105.135) (end 106.955 105.135) (width 0.8) (layer F.Cu) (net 1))
 (segment (start 106.955 105.965) (end 108.145 105.965) (width 0.8) (layer F.Cu) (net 1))
 (segment (start 107.8 106.95) (end 107.8 106.31) (width 0.25) (layer F.Cu) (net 1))
 (segment (start 107.8 106.31) (end 108.145 105.965) (width 0.25) (layer F.Cu) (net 1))
 (segment (start 107.3 106.95) (end 107.3 106.31) (width 0.25) (layer F.Cu) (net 1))
 (segment (start 107.3 106.31) (end 106.955 105.965) (width 0.25) (layer F.Cu) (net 1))
 (segment (start 106.8 106.95) (end 106.8 106.4) (width 0.25) (layer F.Cu) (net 1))
 (segment (start 106.8 106.12) (end 106.955 105.965) (width 0.25) (layer F.Cu) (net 1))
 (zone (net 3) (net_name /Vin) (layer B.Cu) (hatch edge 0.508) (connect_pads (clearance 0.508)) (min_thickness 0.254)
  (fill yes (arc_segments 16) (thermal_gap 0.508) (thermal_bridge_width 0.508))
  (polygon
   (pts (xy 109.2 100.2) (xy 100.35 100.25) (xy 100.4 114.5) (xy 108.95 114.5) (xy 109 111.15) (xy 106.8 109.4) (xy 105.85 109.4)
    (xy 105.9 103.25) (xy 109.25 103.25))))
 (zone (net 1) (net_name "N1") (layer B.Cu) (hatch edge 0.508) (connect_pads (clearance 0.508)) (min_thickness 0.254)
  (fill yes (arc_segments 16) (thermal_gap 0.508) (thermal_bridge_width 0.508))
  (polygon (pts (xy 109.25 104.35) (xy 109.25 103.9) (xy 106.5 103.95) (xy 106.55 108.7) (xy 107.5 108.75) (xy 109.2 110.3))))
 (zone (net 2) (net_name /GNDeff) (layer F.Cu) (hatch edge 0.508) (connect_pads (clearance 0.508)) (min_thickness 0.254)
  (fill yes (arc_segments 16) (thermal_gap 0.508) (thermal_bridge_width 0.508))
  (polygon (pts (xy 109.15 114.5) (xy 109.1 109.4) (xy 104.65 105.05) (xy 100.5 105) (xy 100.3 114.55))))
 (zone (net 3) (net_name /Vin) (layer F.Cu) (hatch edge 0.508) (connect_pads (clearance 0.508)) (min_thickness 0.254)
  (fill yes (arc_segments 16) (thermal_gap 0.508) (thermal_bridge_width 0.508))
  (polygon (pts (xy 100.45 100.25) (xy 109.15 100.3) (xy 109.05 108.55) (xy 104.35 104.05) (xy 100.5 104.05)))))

